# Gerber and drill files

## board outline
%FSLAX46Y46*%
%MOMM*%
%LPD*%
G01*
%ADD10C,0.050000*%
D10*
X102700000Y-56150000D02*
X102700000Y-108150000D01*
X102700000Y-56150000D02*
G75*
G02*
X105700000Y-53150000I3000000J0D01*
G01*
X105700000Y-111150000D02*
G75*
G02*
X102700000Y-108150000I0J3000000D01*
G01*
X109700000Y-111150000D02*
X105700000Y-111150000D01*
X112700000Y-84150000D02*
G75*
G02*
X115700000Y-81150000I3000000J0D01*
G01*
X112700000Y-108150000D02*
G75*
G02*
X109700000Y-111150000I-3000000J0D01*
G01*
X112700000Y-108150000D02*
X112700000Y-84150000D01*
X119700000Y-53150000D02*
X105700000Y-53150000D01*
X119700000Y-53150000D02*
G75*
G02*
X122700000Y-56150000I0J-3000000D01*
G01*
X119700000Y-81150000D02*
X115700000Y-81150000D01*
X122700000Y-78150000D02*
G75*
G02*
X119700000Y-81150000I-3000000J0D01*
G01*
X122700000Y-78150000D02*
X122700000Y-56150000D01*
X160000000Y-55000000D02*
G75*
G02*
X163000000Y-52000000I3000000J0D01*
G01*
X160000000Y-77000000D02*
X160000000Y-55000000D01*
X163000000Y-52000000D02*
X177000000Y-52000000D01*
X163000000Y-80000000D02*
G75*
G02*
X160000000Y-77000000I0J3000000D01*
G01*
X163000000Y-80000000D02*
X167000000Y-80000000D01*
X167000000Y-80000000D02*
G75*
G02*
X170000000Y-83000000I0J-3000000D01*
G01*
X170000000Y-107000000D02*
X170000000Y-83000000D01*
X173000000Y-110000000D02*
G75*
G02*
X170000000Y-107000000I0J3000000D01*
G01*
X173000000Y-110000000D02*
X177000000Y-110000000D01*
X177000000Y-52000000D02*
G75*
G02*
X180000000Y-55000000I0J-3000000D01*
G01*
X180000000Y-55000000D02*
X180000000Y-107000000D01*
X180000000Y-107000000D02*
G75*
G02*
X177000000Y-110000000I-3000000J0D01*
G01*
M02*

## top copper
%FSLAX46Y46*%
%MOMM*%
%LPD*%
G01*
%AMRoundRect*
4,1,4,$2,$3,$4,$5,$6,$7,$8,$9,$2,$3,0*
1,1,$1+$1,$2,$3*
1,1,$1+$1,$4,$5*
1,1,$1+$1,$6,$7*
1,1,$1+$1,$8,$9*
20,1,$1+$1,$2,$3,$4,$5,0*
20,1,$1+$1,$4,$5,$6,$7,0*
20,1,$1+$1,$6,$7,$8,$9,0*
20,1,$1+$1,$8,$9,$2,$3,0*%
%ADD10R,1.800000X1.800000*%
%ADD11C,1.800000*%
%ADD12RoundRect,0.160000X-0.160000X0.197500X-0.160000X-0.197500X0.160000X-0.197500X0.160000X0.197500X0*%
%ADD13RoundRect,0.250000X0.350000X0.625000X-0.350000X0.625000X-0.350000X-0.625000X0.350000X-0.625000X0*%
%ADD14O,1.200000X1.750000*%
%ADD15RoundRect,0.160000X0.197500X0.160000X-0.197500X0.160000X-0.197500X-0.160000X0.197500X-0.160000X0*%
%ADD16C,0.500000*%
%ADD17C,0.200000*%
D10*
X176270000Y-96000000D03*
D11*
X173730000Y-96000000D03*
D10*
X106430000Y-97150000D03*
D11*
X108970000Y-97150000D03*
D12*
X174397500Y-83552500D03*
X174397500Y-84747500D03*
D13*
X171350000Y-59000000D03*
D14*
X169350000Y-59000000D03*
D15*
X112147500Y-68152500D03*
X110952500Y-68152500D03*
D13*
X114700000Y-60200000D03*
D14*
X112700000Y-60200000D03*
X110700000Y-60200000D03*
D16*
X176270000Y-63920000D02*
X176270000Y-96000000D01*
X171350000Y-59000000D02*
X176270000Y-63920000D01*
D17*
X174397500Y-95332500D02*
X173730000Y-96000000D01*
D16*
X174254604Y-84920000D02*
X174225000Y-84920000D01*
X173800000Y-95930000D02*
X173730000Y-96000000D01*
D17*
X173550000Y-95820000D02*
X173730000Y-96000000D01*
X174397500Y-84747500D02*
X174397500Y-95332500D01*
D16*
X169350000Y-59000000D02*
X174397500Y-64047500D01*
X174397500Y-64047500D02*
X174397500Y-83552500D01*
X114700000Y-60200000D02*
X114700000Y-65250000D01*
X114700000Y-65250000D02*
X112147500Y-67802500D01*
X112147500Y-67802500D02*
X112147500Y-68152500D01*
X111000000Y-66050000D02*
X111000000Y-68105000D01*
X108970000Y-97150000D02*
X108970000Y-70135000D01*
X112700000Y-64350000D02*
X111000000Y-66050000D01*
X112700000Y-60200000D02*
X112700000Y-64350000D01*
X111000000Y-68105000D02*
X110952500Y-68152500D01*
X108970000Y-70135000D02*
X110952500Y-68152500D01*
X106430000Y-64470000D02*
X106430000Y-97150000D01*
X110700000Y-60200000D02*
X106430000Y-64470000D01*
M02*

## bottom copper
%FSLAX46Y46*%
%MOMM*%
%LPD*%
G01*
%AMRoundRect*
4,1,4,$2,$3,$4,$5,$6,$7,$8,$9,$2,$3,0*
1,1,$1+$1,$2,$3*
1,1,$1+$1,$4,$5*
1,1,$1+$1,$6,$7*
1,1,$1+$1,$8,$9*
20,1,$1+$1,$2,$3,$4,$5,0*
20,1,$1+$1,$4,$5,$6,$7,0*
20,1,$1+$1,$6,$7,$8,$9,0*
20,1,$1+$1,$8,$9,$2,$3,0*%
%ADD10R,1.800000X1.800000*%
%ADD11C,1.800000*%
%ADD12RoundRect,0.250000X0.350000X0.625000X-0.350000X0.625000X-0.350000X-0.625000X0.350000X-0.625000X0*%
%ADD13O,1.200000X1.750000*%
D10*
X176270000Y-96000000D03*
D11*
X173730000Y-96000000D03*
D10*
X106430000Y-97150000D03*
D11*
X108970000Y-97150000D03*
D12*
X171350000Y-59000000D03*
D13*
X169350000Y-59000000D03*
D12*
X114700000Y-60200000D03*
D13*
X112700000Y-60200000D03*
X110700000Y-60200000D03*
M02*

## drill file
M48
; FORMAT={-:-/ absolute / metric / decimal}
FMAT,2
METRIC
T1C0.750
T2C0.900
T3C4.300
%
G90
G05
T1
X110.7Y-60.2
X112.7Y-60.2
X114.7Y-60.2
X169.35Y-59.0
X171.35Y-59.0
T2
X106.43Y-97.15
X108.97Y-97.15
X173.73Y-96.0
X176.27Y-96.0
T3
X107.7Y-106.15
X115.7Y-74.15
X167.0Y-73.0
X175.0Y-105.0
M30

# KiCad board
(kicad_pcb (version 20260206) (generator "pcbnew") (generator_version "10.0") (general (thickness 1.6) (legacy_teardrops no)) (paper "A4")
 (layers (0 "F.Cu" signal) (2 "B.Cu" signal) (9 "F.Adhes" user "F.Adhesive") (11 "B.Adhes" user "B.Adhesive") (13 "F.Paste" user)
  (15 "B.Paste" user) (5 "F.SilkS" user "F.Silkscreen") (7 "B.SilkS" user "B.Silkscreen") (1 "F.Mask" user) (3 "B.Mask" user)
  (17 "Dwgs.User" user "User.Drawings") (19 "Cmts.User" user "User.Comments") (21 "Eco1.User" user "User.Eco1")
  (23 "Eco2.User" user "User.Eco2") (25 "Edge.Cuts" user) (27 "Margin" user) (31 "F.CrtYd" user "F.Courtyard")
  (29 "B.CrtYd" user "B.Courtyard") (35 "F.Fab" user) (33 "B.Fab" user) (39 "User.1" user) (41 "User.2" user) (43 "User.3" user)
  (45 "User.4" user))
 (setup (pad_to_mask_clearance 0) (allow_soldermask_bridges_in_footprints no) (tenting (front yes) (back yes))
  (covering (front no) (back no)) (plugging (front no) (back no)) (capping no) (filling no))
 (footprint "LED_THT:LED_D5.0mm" (layer "F.Cu") (at 176.27 96 180)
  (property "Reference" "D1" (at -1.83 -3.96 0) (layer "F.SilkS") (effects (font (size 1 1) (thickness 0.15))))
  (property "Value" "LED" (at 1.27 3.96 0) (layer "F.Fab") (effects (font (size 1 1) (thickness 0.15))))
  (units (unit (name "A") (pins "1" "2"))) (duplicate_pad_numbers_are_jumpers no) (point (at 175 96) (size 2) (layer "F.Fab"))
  (pad "1" thru_hole rect (at 0 0 180) (size 1.8 1.8) (drill 0.9) (layers "*.Cu" "*.Mask") (remove_unused_layers no) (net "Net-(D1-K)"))
  (pad "2" thru_hole circle (at 2.54 0 180) (size 1.8 1.8) (drill 0.9) (layers "*.Cu" "*.Mask") (remove_unused_layers no) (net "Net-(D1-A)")))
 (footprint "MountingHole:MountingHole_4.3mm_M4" (layer "F.Cu") (at 175 105)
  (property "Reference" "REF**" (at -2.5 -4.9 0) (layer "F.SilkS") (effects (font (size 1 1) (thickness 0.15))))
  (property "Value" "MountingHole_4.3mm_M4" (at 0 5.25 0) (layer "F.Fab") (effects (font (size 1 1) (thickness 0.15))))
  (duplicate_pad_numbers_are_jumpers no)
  (pad "" np_thru_hole circle (at 0 0) (size 4.3 4.3) (drill 4.3) (layers "*.Cu" "*.Mask")))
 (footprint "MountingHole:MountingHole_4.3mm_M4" (layer "F.Cu") (at 167 73)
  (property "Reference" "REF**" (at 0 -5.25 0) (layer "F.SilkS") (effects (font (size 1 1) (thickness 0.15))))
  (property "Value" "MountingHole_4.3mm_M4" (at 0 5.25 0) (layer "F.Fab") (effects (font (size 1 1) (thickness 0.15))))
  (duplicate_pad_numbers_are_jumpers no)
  (pad "" np_thru_hole circle (at 0 0) (size 4.3 4.3) (drill 4.3) (layers "*.Cu" "*.Mask")))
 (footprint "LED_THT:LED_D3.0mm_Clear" (layer "F.Cu") (at 106.43 97.15)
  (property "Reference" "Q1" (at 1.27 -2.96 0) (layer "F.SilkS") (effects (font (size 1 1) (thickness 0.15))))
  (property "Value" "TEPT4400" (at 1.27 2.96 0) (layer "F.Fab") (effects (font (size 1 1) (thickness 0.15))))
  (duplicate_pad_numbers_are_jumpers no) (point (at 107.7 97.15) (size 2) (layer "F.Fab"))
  (pad "1" thru_hole rect (at 0 0) (size 1.8 1.8) (drill 0.9) (layers "*.Cu" "*.Mask") (remove_unused_layers no) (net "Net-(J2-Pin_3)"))
  (pad "2" thru_hole circle (at 2.54 0) (size 1.8 1.8) (drill 0.9) (layers "*.Cu" "*.Mask") (remove_unused_layers no) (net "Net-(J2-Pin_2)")))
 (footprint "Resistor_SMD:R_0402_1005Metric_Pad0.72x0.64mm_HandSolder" (layer "F.Cu") (at 174.3975 84.15 -90)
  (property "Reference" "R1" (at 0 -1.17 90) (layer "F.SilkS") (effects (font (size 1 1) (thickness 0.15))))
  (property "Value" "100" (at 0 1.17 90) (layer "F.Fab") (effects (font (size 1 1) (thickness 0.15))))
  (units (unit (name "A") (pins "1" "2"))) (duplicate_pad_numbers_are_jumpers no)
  (pad "1" smd roundrect (at -0.5975 0 270) (size 0.715 0.64) (layers "F.Cu" "F.Mask" "F.Paste") (roundrect_rratio 0.25)
   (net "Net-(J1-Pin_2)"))
  (pad "2" smd roundrect (at 0.5975 0 270) (size 0.715 0.64) (layers "F.Cu" "F.Mask" "F.Paste") (roundrect_rratio 0.25) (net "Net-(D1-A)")))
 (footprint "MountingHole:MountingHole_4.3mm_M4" (layer "F.Cu") (at 107.7 106.15)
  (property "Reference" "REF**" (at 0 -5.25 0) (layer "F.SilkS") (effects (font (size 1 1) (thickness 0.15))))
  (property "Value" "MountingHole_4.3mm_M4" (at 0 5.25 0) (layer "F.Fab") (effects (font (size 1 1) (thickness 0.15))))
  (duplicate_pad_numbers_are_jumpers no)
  (pad "" np_thru_hole circle (at 0 0) (size 4.3 4.3) (drill 4.3) (layers "*.Cu" "*.Mask")))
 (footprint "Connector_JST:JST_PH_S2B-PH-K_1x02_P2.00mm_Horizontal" (layer "F.Cu") (at 171.35 59 180)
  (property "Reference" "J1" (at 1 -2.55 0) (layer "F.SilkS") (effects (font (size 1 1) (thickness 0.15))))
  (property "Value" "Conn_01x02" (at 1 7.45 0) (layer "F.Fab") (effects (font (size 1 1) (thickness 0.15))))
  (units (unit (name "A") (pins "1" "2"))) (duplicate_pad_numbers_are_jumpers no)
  (pad "1" thru_hole roundrect (at 0 0 180) (size 1.2 1.75) (drill 0.75) (layers "*.Cu" "*.Mask") (remove_unused_layers no)
   (roundrect_rratio 0.208333) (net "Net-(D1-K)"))
  (pad "2" thru_hole oval (at 2 0 180) (size 1.2 1.75) (drill 0.75) (layers "*.Cu" "*.Mask") (remove_unused_layers no)
   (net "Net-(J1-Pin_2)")))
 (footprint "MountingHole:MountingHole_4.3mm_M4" (layer "F.Cu") (at 115.7 74.15)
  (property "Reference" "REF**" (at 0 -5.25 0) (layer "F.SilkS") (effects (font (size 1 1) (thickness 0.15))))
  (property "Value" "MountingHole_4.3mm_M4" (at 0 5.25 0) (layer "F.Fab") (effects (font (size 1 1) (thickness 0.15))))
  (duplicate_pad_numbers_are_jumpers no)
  (pad "" np_thru_hole circle (at 0 0) (size 4.3 4.3) (drill 4.3) (layers "*.Cu" "*.Mask")))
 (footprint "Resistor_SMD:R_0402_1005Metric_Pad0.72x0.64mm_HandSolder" (layer "F.Cu") (at 111.55 68.1525 180)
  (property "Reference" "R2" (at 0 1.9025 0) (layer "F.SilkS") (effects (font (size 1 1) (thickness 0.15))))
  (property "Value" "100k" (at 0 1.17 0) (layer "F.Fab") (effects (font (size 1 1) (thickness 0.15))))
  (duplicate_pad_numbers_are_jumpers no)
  (pad "1" smd roundrect (at -0.5975 0 180) (size 0.715 0.64) (layers "F.Cu" "F.Mask" "F.Paste") (roundrect_rratio 0.25)
   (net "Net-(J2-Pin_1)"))
  (pad "2" smd roundrect (at 0.5975 0 180) (size 0.715 0.64) (layers "F.Cu" "F.Mask" "F.Paste") (roundrect_rratio 0.25)
   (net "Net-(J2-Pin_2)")))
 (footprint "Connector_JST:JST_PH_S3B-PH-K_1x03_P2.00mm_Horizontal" (layer "F.Cu") (at 114.7 60.2 180)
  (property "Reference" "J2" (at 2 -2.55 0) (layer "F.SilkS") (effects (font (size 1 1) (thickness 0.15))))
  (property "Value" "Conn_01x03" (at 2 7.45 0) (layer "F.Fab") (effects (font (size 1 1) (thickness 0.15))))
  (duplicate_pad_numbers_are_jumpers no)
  (pad "1" thru_hole roundrect (at 0 0 180) (size 1.2 1.75) (drill 0.75) (layers "*.Cu" "*.Mask") (remove_unused_layers no)
   (roundrect_rratio 0.208333) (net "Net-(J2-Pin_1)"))
  (pad "2" thru_hole oval (at 2 0 180) (size 1.2 1.75) (drill 0.75) (layers "*.Cu" "*.Mask") (remove_unused_layers no)
   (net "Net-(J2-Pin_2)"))
  (pad "3" thru_hole oval (at 4 0 180) (size 1.2 1.75) (drill 0.75) (layers "*.Cu" "*.Mask") (remove_unused_layers no)
   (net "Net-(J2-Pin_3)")))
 (gr_line (start 102.7 56.15) (end 102.7 108.15) (stroke (width 0.05) (type default)) (layer "Edge.Cuts"))
 (gr_arc (start 102.7 56.15) (mid 103.57868 54.02868) (end 105.7 53.15) (stroke (width 0.05) (type default)) (layer "Edge.Cuts"))
 (gr_arc (start 105.7 111.15) (mid 103.57868 110.27132) (end 102.7 108.15) (stroke (width 0.05) (type default)) (layer "Edge.Cuts"))
 (gr_line (start 109.7 111.15) (end 105.7 111.15) (stroke (width 0.05) (type default)) (layer "Edge.Cuts"))
 (gr_arc (start 112.7 84.15) (mid 113.57868 82.02868) (end 115.7 81.15) (stroke (width 0.05) (type default)) (layer "Edge.Cuts"))
 (gr_arc (start 112.7 108.15) (mid 111.82132 110.27132) (end 109.7 111.15) (stroke (width 0.05) (type default)) (layer "Edge.Cuts"))
 (gr_line (start 112.7 108.15) (end 112.7 84.15) (stroke (width 0.05) (type default)) (layer "Edge.Cuts"))
 (gr_line (start 119.7 53.15) (end 105.7 53.15) (stroke (width 0.05) (type solid)) (layer "Edge.Cuts"))
 (gr_arc (start 119.7 53.15) (mid 121.82132 54.02868) (end 122.7 56.15) (stroke (width 0.05) (type default)) (layer "Edge.Cuts"))
 (gr_line (start 119.7 81.15) (end 115.7 81.15) (stroke (width 0.05) (type default)) (layer "Edge.Cuts"))
 (gr_arc (start 122.7 78.15) (mid 121.82132 80.27132) (end 119.7 81.15) (stroke (width 0.05) (type default)) (layer "Edge.Cuts"))
 (gr_line (start 122.7 78.15) (end 122.7 56.15) (stroke (width 0.05) (type default)) (layer "Edge.Cuts"))
 (gr_arc (start 160 55) (mid 160.87868 52.87868) (end 163 52) (stroke (width 0.05) (type default)) (layer "Edge.Cuts"))
 (gr_line (start 160 77) (end 160 55) (stroke (width 0.05) (type default)) (layer "Edge.Cuts"))
 (gr_line (start 163 52) (end 177 52) (stroke (width 0.05) (type solid)) (layer "Edge.Cuts"))
 (gr_arc (start 163 80) (mid 160.87868 79.12132) (end 160 77) (stroke (width 0.05) (type default)) (layer "Edge.Cuts"))
 (gr_line (start 163 80) (end 167 80) (stroke (width 0.05) (type default)) (layer "Edge.Cuts"))
 (gr_arc (start 167 80) (mid 169.12132 80.87868) (end 170 83) (stroke (width 0.05) (type default)) (layer "Edge.Cuts"))
 (gr_line (start 170 107) (end 170 83) (stroke (width 0.05) (type default)) (layer "Edge.Cuts"))
 (gr_arc (start 173 110) (mid 170.87868 109.12132) (end 170 107) (stroke (width 0.05) (type default)) (layer "Edge.Cuts"))
 (gr_line (start 173 110) (end 177 110) (stroke (width 0.05) (type default)) (layer "Edge.Cuts"))
 (gr_arc (start 177 52) (mid 179.12132 52.87868) (end 180 55) (stroke (width 0.05) (type default)) (layer "Edge.Cuts"))
 (gr_line (start 180 55) (end 180 107) (stroke (width 0.05) (type default)) (layer "Edge.Cuts"))
 (gr_arc (start 180 107) (mid 179.12132 109.12132) (end 177 110) (stroke (width 0.05) (type default)) (layer "Edge.Cuts"))
 (segment (start 176.27 63.92) (end 176.27 96) (width 0.5) (layer "F.Cu") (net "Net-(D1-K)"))
 (segment (start 171.35 59) (end 176.27 63.92) (width 0.5) (layer "F.Cu") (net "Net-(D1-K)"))
 (segment (start 174.3975 95.3325) (end 173.73 96) (width 0.2) (layer "F.Cu") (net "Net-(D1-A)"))
 (segment (start 174.254604 84.92) (end 174.225 84.92) (width 0.5) (layer "F.Cu") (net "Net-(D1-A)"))
 (segment (start 173.8 95.93) (end 173.73 96) (width 0.5) (layer "F.Cu") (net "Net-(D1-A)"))
 (segment (start 173.55 95.82) (end 173.73 96) (width 0.2) (layer "F.Cu") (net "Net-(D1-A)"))
 (segment (start 174.3975 84.7475) (end 174.3975 95.3325) (width 0.2) (layer "F.Cu") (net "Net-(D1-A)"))
 (segment (start 169.35 59) (end 174.3975 64.0475) (width 0.5) (layer "F.Cu") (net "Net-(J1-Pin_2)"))
 (segment (start 174.3975 64.0475) (end 174.3975 83.5525) (width 0.5) (layer "F.Cu") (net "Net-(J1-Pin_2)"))
 (segment (start 114.7 60.2) (end 114.7 65.25) (width 0.5) (layer "F.Cu") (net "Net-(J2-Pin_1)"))
 (segment (start 114.7 65.25) (end 112.1475 67.8025) (width 0.5) (layer "F.Cu") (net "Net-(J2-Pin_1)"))
 (segment (start 112.1475 67.8025) (end 112.1475 68.1525) (width 0.5) (layer "F.Cu") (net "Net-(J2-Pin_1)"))
 (segment (start 111 66.05) (end 111 68.105) (width 0.5) (layer "F.Cu") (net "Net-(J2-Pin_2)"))
 (segment (start 108.97 97.15) (end 108.97 70.135) (width 0.5) (layer "F.Cu") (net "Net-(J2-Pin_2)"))
 (segment (start 112.7 64.35) (end 111 66.05) (width 0.5) (layer "F.Cu") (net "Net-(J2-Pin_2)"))
 (segment (start 112.7 60.2) (end 112.7 64.35) (width 0.5) (layer "F.Cu") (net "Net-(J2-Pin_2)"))
 (segment (start 111 68.105) (end 110.9525 68.1525) (width 0.5) (layer "F.Cu") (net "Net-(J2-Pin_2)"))
 (segment (start 108.97 70.135) (end 110.9525 68.1525) (width 0.5) (layer "F.Cu") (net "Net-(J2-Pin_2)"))
 (segment (start 106.43 64.47) (end 106.43 97.15) (width 0.5) (layer "F.Cu") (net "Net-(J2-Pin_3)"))
 (segment (start 110.7 60.2) (end 106.43 64.47) (width 0.5) (layer "F.Cu") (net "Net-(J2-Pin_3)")))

